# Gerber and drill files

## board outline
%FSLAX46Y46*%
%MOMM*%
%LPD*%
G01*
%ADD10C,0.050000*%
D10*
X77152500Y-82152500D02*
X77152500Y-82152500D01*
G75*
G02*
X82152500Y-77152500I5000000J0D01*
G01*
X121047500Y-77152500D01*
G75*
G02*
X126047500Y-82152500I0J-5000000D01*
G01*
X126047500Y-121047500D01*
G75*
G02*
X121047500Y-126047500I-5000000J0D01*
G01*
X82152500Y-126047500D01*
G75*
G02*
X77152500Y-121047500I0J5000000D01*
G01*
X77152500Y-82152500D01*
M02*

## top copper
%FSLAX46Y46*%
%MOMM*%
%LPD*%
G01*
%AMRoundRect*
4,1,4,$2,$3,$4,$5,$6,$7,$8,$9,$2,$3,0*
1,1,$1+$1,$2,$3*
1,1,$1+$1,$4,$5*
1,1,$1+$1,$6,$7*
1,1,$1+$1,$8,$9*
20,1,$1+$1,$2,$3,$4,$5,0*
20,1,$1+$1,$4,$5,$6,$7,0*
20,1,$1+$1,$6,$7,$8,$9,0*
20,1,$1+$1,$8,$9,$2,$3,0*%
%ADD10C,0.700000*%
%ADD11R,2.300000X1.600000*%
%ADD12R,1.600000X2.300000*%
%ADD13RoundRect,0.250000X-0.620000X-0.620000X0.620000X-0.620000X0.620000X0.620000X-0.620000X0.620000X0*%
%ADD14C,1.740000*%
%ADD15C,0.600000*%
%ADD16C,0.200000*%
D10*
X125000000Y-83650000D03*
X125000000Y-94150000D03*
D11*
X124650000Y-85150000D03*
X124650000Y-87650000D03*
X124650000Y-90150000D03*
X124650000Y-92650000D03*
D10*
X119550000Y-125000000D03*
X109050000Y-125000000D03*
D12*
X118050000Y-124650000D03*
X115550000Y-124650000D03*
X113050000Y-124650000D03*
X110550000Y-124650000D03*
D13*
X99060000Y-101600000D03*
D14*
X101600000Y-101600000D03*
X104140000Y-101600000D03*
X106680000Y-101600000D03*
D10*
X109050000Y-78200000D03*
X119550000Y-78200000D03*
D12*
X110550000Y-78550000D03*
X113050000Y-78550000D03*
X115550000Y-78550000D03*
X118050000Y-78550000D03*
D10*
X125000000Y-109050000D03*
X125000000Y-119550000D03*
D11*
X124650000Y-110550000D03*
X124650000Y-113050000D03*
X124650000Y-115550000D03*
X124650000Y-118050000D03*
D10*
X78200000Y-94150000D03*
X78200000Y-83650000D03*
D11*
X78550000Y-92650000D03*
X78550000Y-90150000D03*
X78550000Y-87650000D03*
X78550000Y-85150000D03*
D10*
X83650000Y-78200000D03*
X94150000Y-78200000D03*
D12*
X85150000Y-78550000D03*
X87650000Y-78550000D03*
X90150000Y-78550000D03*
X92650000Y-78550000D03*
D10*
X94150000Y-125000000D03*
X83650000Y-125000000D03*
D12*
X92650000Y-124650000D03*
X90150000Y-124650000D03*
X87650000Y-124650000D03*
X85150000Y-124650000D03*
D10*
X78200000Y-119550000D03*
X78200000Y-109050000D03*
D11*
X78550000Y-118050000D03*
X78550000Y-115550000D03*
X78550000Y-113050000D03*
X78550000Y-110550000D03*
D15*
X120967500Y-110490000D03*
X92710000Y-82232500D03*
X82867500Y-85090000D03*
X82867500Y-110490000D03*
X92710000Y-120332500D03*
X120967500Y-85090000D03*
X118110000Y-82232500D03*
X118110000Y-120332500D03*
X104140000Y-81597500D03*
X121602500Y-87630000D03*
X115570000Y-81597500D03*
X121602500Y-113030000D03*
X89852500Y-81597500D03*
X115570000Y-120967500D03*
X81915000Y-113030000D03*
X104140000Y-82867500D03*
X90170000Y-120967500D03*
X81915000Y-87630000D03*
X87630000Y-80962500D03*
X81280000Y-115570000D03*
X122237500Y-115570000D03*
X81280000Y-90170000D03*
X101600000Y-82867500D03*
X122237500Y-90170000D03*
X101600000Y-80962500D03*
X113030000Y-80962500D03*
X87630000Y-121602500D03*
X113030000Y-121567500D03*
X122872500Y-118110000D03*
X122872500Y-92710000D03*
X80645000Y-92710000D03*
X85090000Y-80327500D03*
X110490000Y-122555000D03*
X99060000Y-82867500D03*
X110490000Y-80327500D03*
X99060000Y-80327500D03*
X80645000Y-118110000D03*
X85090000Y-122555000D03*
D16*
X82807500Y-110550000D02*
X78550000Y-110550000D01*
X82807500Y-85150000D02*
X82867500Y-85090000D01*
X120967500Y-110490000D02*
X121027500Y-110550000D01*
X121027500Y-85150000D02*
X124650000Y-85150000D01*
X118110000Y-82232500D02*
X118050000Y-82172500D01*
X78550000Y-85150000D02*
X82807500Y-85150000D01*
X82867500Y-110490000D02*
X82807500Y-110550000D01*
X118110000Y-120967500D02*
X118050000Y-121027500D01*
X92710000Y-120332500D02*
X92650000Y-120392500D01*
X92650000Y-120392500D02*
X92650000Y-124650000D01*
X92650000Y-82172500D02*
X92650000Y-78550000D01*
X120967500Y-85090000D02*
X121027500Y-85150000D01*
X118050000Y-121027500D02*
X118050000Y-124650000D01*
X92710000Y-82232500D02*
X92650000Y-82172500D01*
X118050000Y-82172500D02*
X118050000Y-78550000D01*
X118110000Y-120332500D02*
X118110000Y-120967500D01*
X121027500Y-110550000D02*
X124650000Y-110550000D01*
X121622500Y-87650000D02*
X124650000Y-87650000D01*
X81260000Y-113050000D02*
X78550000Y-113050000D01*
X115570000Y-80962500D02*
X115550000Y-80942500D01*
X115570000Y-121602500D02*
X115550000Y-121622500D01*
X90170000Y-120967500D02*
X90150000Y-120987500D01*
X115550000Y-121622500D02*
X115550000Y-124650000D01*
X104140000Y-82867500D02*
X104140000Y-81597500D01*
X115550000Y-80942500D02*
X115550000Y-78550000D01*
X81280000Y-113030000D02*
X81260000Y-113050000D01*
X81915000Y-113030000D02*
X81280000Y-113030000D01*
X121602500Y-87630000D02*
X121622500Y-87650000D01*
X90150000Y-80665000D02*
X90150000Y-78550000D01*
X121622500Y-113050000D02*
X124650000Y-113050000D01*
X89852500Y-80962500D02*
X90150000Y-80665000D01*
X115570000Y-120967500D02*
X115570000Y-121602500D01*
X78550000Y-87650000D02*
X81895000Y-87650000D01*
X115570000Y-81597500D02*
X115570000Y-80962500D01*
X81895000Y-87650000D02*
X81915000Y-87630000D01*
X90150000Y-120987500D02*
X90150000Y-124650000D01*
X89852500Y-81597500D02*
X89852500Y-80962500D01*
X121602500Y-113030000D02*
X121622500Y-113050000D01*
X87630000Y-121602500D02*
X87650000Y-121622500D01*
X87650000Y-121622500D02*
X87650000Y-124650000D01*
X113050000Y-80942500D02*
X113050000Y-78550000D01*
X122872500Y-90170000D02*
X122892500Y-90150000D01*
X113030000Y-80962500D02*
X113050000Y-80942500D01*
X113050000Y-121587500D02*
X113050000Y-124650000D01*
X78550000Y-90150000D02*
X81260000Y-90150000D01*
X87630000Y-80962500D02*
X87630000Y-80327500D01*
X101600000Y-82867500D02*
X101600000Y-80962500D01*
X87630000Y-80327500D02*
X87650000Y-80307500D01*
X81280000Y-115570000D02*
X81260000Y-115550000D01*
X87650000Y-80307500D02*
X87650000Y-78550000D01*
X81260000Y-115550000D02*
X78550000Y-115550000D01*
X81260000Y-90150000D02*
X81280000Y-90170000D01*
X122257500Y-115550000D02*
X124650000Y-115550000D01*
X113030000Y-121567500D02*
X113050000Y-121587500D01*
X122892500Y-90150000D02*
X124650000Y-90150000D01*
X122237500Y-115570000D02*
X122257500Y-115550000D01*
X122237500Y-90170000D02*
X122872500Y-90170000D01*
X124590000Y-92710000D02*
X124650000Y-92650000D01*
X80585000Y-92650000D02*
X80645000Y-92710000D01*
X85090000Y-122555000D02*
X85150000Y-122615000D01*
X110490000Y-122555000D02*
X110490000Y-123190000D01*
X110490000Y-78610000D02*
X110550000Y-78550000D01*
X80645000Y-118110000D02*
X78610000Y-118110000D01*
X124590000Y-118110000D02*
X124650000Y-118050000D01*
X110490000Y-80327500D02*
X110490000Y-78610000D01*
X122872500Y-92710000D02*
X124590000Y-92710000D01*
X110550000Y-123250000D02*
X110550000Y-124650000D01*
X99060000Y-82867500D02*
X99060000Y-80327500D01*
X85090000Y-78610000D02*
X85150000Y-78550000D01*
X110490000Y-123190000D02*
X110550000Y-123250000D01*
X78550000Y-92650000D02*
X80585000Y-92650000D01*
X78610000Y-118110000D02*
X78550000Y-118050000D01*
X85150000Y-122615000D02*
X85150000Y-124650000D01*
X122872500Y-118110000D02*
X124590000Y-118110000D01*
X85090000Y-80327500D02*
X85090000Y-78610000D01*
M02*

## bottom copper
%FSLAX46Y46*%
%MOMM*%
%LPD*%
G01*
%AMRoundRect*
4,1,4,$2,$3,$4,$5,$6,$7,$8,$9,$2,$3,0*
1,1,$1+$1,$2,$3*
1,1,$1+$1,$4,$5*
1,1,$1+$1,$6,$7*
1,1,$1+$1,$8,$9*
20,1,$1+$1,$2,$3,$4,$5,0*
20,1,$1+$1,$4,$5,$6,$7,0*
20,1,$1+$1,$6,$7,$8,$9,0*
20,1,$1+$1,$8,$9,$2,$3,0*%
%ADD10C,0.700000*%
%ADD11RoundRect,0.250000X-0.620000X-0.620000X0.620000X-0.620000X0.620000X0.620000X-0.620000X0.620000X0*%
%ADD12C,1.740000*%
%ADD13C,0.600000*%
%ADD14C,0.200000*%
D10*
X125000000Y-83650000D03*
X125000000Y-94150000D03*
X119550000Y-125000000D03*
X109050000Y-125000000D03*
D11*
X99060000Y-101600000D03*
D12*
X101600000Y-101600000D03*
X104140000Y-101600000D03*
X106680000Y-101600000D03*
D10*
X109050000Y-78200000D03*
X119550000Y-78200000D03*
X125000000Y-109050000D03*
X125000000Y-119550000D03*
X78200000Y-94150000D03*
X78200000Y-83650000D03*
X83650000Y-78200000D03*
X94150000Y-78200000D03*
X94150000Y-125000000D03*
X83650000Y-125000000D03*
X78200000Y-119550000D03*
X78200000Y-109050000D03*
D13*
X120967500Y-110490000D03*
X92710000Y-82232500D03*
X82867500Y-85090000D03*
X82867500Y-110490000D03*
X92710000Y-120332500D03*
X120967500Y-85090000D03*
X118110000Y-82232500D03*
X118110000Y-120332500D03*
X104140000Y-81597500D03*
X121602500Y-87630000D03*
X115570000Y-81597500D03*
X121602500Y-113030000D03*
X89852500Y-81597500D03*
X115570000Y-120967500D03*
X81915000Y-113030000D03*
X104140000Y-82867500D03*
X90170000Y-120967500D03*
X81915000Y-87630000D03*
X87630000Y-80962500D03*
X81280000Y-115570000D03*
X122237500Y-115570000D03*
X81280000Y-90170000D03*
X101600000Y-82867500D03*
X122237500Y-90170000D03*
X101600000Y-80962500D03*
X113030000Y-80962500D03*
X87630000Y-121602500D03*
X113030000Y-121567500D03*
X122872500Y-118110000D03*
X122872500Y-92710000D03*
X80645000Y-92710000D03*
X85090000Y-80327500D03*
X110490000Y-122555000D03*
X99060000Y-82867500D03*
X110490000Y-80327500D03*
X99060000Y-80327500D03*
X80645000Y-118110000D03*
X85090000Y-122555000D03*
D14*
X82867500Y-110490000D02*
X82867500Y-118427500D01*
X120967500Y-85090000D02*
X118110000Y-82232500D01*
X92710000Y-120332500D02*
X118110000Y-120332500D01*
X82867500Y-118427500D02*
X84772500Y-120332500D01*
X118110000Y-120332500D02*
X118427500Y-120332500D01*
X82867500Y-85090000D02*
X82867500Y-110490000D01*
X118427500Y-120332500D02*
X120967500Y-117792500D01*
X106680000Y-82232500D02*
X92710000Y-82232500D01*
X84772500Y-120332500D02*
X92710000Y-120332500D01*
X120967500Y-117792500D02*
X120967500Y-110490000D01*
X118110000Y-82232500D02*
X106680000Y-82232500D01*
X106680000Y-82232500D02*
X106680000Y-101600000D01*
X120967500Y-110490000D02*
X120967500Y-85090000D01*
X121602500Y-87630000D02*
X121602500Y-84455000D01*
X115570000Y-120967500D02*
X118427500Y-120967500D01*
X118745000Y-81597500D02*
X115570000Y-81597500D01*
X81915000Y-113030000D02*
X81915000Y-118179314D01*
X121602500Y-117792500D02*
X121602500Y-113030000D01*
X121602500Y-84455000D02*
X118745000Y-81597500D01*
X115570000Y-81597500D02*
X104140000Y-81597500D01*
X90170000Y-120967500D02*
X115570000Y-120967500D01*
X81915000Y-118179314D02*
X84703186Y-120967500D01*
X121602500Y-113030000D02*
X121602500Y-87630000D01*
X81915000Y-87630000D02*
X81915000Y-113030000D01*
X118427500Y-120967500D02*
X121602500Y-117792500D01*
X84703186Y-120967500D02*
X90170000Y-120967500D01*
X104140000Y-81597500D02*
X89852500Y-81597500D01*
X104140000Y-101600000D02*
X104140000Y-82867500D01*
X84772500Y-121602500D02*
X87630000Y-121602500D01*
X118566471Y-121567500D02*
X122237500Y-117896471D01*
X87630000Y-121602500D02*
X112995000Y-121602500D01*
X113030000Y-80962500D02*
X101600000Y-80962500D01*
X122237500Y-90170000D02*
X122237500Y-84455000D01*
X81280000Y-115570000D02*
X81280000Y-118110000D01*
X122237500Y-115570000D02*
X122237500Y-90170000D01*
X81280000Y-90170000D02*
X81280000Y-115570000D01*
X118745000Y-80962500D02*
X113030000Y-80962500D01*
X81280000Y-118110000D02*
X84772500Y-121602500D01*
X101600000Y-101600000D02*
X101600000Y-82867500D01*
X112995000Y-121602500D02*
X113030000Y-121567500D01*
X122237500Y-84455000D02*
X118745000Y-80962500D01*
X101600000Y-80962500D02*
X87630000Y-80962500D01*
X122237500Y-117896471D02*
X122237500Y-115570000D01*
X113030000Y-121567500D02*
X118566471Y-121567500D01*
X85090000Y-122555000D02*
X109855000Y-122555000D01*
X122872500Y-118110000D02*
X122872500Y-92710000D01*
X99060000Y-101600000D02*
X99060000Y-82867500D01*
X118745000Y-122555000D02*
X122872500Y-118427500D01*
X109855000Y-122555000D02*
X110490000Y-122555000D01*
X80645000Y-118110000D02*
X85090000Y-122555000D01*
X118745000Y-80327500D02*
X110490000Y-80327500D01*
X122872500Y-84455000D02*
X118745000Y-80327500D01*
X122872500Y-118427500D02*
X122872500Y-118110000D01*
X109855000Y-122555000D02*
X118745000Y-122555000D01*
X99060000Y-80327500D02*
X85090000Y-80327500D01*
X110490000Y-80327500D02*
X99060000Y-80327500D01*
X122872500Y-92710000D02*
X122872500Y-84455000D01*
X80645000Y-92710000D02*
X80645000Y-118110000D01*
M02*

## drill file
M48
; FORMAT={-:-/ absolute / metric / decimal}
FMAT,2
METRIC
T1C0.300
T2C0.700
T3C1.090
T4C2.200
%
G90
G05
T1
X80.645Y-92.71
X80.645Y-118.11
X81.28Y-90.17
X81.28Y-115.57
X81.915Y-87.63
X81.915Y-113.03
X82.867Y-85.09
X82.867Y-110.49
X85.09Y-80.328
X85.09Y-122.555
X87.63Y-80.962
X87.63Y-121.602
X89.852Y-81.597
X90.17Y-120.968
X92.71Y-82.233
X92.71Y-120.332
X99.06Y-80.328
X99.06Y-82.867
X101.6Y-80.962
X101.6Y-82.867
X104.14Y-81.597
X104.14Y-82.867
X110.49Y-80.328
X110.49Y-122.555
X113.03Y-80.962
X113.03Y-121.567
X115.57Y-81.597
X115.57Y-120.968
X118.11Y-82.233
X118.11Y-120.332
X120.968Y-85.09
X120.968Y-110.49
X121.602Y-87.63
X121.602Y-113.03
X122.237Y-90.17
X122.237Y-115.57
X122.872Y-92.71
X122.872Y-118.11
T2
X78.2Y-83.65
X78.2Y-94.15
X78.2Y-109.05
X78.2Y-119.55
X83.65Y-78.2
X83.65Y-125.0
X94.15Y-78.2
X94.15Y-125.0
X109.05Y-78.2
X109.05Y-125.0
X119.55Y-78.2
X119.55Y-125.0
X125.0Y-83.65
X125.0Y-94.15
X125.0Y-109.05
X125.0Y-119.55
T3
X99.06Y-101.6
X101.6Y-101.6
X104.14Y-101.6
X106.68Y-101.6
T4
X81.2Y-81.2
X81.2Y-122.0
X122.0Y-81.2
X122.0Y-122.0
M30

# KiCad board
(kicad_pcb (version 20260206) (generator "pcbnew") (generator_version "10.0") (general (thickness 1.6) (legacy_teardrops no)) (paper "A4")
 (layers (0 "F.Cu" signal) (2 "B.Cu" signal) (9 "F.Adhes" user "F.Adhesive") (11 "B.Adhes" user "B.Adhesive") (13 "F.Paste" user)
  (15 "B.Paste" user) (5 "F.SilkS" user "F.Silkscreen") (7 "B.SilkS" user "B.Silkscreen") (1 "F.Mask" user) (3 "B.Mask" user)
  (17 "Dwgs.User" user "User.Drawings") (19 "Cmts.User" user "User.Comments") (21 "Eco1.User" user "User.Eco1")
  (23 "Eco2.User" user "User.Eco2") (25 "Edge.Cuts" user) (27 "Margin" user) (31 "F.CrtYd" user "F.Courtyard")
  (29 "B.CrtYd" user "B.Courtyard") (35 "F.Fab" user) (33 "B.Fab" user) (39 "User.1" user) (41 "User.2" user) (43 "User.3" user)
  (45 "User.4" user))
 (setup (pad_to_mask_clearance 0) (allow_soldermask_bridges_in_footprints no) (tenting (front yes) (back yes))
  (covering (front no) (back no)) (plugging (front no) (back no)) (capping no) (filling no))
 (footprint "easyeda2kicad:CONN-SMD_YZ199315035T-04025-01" (layer "F.Cu") (at 124.65 88.9 -90)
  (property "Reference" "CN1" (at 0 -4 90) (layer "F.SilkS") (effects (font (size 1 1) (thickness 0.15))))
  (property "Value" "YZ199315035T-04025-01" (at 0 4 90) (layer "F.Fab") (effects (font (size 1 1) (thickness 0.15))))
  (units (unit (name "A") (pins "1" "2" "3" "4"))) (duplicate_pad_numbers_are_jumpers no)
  (pad "" thru_hole circle (at -5.25 -0.35 270) (size 0.7 0.7) (drill 0.7) (layers "*.Cu" "*.Mask") (remove_unused_layers no))
  (pad "" thru_hole circle (at 5.25 -0.35 270) (size 0.7 0.7) (drill 0.7) (layers "*.Cu" "*.Mask") (remove_unused_layers no))
  (pad "1" smd rect (at -3.75 0 270) (size 1.6 2.3) (layers "F.Cu" "F.Mask" "F.Paste") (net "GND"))
  (pad "2" smd rect (at -1.25 0 270) (size 1.6 2.3) (layers "F.Cu" "F.Mask" "F.Paste") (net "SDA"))
  (pad "3" smd rect (at 1.25 0 270) (size 1.6 2.3) (layers "F.Cu" "F.Mask" "F.Paste") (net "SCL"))
  (pad "4" smd rect (at 3.75 0 270) (size 1.6 2.3) (layers "F.Cu" "F.Mask" "F.Paste") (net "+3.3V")))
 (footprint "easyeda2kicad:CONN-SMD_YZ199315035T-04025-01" (layer "F.Cu") (at 114.3 124.65 180)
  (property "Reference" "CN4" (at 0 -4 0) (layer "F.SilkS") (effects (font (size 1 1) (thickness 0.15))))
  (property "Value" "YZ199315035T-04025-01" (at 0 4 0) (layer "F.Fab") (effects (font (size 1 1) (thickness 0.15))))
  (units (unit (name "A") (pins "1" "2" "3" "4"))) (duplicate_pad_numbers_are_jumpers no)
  (pad "" thru_hole circle (at -5.25 -0.35 180) (size 0.7 0.7) (drill 0.7) (layers "*.Cu" "*.Mask") (remove_unused_layers no))
  (pad "" thru_hole circle (at 5.25 -0.35 180) (size 0.7 0.7) (drill 0.7) (layers "*.Cu" "*.Mask") (remove_unused_layers no))
  (pad "1" smd rect (at -3.75 0 180) (size 1.6 2.3) (layers "F.Cu" "F.Mask" "F.Paste") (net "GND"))
  (pad "2" smd rect (at -1.25 0 180) (size 1.6 2.3) (layers "F.Cu" "F.Mask" "F.Paste") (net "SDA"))
  (pad "3" smd rect (at 1.25 0 180) (size 1.6 2.3) (layers "F.Cu" "F.Mask" "F.Paste") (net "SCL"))
  (pad "4" smd rect (at 3.75 0 180) (size 1.6 2.3) (layers "F.Cu" "F.Mask" "F.Paste") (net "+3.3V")))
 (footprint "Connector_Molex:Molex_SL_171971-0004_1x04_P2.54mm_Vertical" (layer "F.Cu") (at 99.06 101.6)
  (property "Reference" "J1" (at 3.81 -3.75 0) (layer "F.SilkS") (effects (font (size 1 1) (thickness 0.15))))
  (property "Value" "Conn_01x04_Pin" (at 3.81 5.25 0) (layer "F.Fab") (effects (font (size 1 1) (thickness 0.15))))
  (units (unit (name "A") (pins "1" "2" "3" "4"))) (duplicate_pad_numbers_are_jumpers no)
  (pad "1" thru_hole roundrect (at 0 0) (size 1.74 1.74) (drill 1.09) (layers "*.Cu" "*.Mask") (remove_unused_layers no)
   (roundrect_rratio 0.143678) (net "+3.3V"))
  (pad "2" thru_hole circle (at 2.54 0) (size 1.74 1.74) (drill 1.09) (layers "*.Cu" "*.Mask") (remove_unused_layers no) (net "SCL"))
  (pad "3" thru_hole circle (at 5.08 0) (size 1.74 1.74) (drill 1.09) (layers "*.Cu" "*.Mask") (remove_unused_layers no) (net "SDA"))
  (pad "4" thru_hole circle (at 7.62 0) (size 1.74 1.74) (drill 1.09) (layers "*.Cu" "*.Mask") (remove_unused_layers no) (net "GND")))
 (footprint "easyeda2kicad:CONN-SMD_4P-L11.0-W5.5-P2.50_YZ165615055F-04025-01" (layer "F.Cu") (at 114.3 78.55)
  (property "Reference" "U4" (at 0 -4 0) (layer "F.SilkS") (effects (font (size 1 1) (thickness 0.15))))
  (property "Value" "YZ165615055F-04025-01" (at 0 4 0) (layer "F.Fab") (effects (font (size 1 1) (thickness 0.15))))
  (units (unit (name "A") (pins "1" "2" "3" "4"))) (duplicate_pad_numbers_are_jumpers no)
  (pad "" thru_hole circle (at -5.25 -0.35) (size 0.7 0.7) (drill 0.7) (layers "*.Cu" "*.Mask") (remove_unused_layers no))
  (pad "" thru_hole circle (at 5.25 -0.35) (size 0.7 0.7) (drill 0.7) (layers "*.Cu" "*.Mask") (remove_unused_layers no))
  (pad "1" smd rect (at -3.75 0) (size 1.6 2.3) (layers "F.Cu" "F.Mask" "F.Paste") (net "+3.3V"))
  (pad "2" smd rect (at -1.25 0) (size 1.6 2.3) (layers "F.Cu" "F.Mask" "F.Paste") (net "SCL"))
  (pad "3" smd rect (at 1.25 0) (size 1.6 2.3) (layers "F.Cu" "F.Mask" "F.Paste") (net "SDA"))
  (pad "4" smd rect (at 3.75 0) (size 1.6 2.3) (layers "F.Cu" "F.Mask" "F.Paste") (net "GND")))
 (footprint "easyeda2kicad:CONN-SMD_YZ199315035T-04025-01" (layer "F.Cu") (at 124.65 114.3 -90)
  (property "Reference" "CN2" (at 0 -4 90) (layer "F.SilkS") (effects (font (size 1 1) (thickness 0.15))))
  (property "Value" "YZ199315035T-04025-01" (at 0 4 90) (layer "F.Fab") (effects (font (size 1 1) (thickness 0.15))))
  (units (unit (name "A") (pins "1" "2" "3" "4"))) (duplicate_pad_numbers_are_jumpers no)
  (pad "" thru_hole circle (at -5.25 -0.35 270) (size 0.7 0.7) (drill 0.7) (layers "*.Cu" "*.Mask") (remove_unused_layers no))
  (pad "" thru_hole circle (at 5.25 -0.35 270) (size 0.7 0.7) (drill 0.7) (layers "*.Cu" "*.Mask") (remove_unused_layers no))
  (pad "1" smd rect (at -3.75 0 270) (size 1.6 2.3) (layers "F.Cu" "F.Mask" "F.Paste") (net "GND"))
  (pad "2" smd rect (at -1.25 0 270) (size 1.6 2.3) (layers "F.Cu" "F.Mask" "F.Paste") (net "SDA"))
  (pad "3" smd rect (at 1.25 0 270) (size 1.6 2.3) (layers "F.Cu" "F.Mask" "F.Paste") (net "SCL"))
  (pad "4" smd rect (at 3.75 0 270) (size 1.6 2.3) (layers "F.Cu" "F.Mask" "F.Paste") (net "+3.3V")))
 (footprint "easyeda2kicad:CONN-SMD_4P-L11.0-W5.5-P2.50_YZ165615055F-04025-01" (layer "F.Cu") (at 78.55 88.9 90)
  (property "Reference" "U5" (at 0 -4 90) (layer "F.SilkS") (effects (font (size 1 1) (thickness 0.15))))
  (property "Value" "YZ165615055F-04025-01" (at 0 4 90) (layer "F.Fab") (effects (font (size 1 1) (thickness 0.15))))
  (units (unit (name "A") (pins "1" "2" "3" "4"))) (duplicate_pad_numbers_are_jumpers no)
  (pad "" thru_hole circle (at -5.25 -0.35 90) (size 0.7 0.7) (drill 0.7) (layers "*.Cu" "*.Mask") (remove_unused_layers no))
  (pad "" thru_hole circle (at 5.25 -0.35 90) (size 0.7 0.7) (drill 0.7) (layers "*.Cu" "*.Mask") (remove_unused_layers no))
  (pad "1" smd rect (at -3.75 0 90) (size 1.6 2.3) (layers "F.Cu" "F.Mask" "F.Paste") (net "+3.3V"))
  (pad "2" smd rect (at -1.25 0 90) (size 1.6 2.3) (layers "F.Cu" "F.Mask" "F.Paste") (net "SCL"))
  (pad "3" smd rect (at 1.25 0 90) (size 1.6 2.3) (layers "F.Cu" "F.Mask" "F.Paste") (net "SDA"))
  (pad "4" smd rect (at 3.75 0 90) (size 1.6 2.3) (layers "F.Cu" "F.Mask" "F.Paste") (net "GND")))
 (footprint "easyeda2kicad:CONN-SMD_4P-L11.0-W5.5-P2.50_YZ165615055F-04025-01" (layer "F.Cu") (at 88.9 78.55)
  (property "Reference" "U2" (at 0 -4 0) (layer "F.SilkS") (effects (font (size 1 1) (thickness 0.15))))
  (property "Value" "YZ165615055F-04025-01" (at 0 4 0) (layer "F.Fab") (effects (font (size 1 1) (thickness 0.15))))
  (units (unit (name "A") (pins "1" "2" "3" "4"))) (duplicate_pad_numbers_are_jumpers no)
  (pad "" thru_hole circle (at -5.25 -0.35) (size 0.7 0.7) (drill 0.7) (layers "*.Cu" "*.Mask") (remove_unused_layers no))
  (pad "" thru_hole circle (at 5.25 -0.35) (size 0.7 0.7) (drill 0.7) (layers "*.Cu" "*.Mask") (remove_unused_layers no))
  (pad "1" smd rect (at -3.75 0) (size 1.6 2.3) (layers "F.Cu" "F.Mask" "F.Paste") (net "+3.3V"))
  (pad "2" smd rect (at -1.25 0) (size 1.6 2.3) (layers "F.Cu" "F.Mask" "F.Paste") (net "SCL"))
  (pad "3" smd rect (at 1.25 0) (size 1.6 2.3) (layers "F.Cu" "F.Mask" "F.Paste") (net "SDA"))
  (pad "4" smd rect (at 3.75 0) (size 1.6 2.3) (layers "F.Cu" "F.Mask" "F.Paste") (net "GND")))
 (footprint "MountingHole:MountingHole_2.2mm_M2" (layer "F.Cu") (at 122 81.2)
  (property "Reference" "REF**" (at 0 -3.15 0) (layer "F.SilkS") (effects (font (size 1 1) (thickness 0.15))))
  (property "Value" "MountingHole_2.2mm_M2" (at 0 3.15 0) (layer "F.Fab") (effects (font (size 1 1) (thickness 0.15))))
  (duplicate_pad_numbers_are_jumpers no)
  (pad "" np_thru_hole circle (at 0 0) (size 2.2 2.2) (drill 2.2) (layers "*.Cu" "*.Mask")))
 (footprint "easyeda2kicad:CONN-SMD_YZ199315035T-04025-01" (layer "F.Cu") (at 88.9 124.65 180)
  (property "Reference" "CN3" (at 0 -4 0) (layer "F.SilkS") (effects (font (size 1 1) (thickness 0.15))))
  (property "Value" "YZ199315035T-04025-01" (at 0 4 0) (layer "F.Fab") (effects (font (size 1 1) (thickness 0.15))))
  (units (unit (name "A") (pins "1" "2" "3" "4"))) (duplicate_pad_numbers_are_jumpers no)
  (pad "" thru_hole circle (at -5.25 -0.35 180) (size 0.7 0.7) (drill 0.7) (layers "*.Cu" "*.Mask") (remove_unused_layers no))
  (pad "" thru_hole circle (at 5.25 -0.35 180) (size 0.7 0.7) (drill 0.7) (layers "*.Cu" "*.Mask") (remove_unused_layers no))
  (pad "1" smd rect (at -3.75 0 180) (size 1.6 2.3) (layers "F.Cu" "F.Mask" "F.Paste") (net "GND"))
  (pad "2" smd rect (at -1.25 0 180) (size 1.6 2.3) (layers "F.Cu" "F.Mask" "F.Paste") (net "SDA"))
  (pad "3" smd rect (at 1.25 0 180) (size 1.6 2.3) (layers "F.Cu" "F.Mask" "F.Paste") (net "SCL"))
  (pad "4" smd rect (at 3.75 0 180) (size 1.6 2.3) (layers "F.Cu" "F.Mask" "F.Paste") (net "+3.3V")))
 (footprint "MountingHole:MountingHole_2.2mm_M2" (layer "F.Cu") (at 81.2 81.2)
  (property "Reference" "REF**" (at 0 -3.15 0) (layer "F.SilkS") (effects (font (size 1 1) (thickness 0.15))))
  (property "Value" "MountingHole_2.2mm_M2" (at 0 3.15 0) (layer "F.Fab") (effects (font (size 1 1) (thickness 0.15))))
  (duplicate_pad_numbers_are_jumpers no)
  (pad "" np_thru_hole circle (at 0 0) (size 2.2 2.2) (drill 2.2) (layers "*.Cu" "*.Mask")))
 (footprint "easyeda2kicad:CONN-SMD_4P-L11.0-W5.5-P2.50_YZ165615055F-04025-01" (layer "F.Cu") (at 78.55 114.3 90)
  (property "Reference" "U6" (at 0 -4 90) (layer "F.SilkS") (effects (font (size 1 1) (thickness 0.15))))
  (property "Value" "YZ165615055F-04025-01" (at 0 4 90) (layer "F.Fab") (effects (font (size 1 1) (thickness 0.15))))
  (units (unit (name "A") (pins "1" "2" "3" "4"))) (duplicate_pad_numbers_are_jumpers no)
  (pad "" thru_hole circle (at -5.25 -0.35 90) (size 0.7 0.7) (drill 0.7) (layers "*.Cu" "*.Mask") (remove_unused_layers no))
  (pad "" thru_hole circle (at 5.25 -0.35 90) (size 0.7 0.7) (drill 0.7) (layers "*.Cu" "*.Mask") (remove_unused_layers no))
  (pad "1" smd rect (at -3.75 0 90) (size 1.6 2.3) (layers "F.Cu" "F.Mask" "F.Paste") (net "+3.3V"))
  (pad "2" smd rect (at -1.25 0 90) (size 1.6 2.3) (layers "F.Cu" "F.Mask" "F.Paste") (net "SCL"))
  (pad "3" smd rect (at 1.25 0 90) (size 1.6 2.3) (layers "F.Cu" "F.Mask" "F.Paste") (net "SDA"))
  (pad "4" smd rect (at 3.75 0 90) (size 1.6 2.3) (layers "F.Cu" "F.Mask" "F.Paste") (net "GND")))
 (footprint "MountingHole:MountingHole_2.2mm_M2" (layer "F.Cu") (at 81.2 122)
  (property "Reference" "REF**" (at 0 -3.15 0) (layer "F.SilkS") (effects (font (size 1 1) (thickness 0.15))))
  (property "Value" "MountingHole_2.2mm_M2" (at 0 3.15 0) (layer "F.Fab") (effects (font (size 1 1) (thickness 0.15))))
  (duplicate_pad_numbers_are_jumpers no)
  (pad "" np_thru_hole circle (at 0 0) (size 2.2 2.2) (drill 2.2) (layers "*.Cu" "*.Mask")))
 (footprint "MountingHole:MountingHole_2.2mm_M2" (layer "F.Cu") (at 122 122)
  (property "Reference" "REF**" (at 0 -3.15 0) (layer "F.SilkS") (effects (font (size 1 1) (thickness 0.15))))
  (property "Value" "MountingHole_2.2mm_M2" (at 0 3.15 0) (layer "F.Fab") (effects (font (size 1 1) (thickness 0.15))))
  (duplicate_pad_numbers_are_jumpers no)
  (pad "" np_thru_hole circle (at 0 0) (size 2.2 2.2) (drill 2.2) (layers "*.Cu" "*.Mask")))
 (gr_rect (start 77.1525 77.1525) (end 126.0475 126.0475) (radius 5) (stroke (width 0.05) (type solid)) (fill no) (layer "Edge.Cuts"))
 (segment (start 82.8075 110.55) (end 78.55 110.55) (width 0.2) (layer "F.Cu") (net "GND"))
 (segment (start 82.8075 85.15) (end 82.8675 85.09) (width 0.2) (layer "F.Cu") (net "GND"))
 (segment (start 120.9675 110.49) (end 121.0275 110.55) (width 0.2) (layer "F.Cu") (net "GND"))
 (segment (start 121.0275 85.15) (end 124.65 85.15) (width 0.2) (layer "F.Cu") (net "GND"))
 (segment (start 118.11 82.2325) (end 118.05 82.1725) (width 0.2) (layer "F.Cu") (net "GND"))
 (segment (start 78.55 85.15) (end 82.8075 85.15) (width 0.2) (layer "F.Cu") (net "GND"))
 (segment (start 82.8675 110.49) (end 82.8075 110.55) (width 0.2) (layer "F.Cu") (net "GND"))
 (segment (start 118.11 120.9675) (end 118.05 121.0275) (width 0.2) (layer "F.Cu") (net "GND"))
 (segment (start 92.71 120.3325) (end 92.65 120.3925) (width 0.2) (layer "F.Cu") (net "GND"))
 (segment (start 92.65 120.3925) (end 92.65 124.65) (width 0.2) (layer "F.Cu") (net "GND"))
 (segment (start 92.65 82.1725) (end 92.65 78.55) (width 0.2) (layer "F.Cu") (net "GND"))
 (segment (start 120.9675 85.09) (end 121.0275 85.15) (width 0.2) (layer "F.Cu") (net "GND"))
 (segment (start 118.05 121.0275) (end 118.05 124.65) (width 0.2) (layer "F.Cu") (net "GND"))
 (segment (start 92.71 82.2325) (end 92.65 82.1725) (width 0.2) (layer "F.Cu") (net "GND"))
 (segment (start 118.05 82.1725) (end 118.05 78.55) (width 0.2) (layer "F.Cu") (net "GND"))
 (segment (start 118.11 120.3325) (end 118.11 120.9675) (width 0.2) (layer "F.Cu") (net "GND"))
 (segment (start 121.0275 110.55) (end 124.65 110.55) (width 0.2) (layer "F.Cu") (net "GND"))
 (via (at 120.9675 110.49) (size 0.6) (drill 0.3) (layers "F.Cu" "B.Cu") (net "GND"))
 (via (at 92.71 82.2325) (size 0.6) (drill 0.3) (layers "F.Cu" "B.Cu") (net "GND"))
 (via (at 82.8675 85.09) (size 0.6) (drill 0.3) (layers "F.Cu" "B.Cu") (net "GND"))
 (via (at 82.8675 110.49) (size 0.6) (drill 0.3) (layers "F.Cu" "B.Cu") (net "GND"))
 (via (at 92.71 120.3325) (size 0.6) (drill 0.3) (layers "F.Cu" "B.Cu") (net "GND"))
 (via (at 120.9675 85.09) (size 0.6) (drill 0.3) (layers "F.Cu" "B.Cu") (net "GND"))
 (via (at 118.11 82.2325) (size 0.6) (drill 0.3) (layers "F.Cu" "B.Cu") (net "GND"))
 (via (at 118.11 120.3325) (size 0.6) (drill 0.3) (layers "F.Cu" "B.Cu") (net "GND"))
 (segment (start 82.8675 110.49) (end 82.8675 118.4275) (width 0.2) (layer "B.Cu") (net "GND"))
 (segment (start 120.9675 85.09) (end 118.11 82.2325) (width 0.2) (layer "B.Cu") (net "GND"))
 (segment (start 92.71 120.3325) (end 118.11 120.3325) (width 0.2) (layer "B.Cu") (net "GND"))
 (segment (start 82.8675 118.4275) (end 84.7725 120.3325) (width 0.2) (layer "B.Cu") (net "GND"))
 (segment (start 118.11 120.3325) (end 118.4275 120.3325) (width 0.2) (layer "B.Cu") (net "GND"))
 (segment (start 82.8675 85.09) (end 82.8675 110.49) (width 0.2) (layer "B.Cu") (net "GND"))
 (segment (start 118.4275 120.3325) (end 120.9675 117.7925) (width 0.2) (layer "B.Cu") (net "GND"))
 (segment (start 106.68 82.2325) (end 92.71 82.2325) (width 0.2) (layer "B.Cu") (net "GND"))
 (segment (start 84.7725 120.3325) (end 92.71 120.3325) (width 0.2) (layer "B.Cu") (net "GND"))
 (segment (start 120.9675 117.7925) (end 120.9675 110.49) (width 0.2) (layer "B.Cu") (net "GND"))
 (segment (start 118.11 82.2325) (end 106.68 82.2325) (width 0.2) (layer "B.Cu") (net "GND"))
 (segment (start 106.68 82.2325) (end 106.68 101.6) (width 0.2) (layer "B.Cu") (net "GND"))
 (segment (start 120.9675 110.49) (end 120.9675 85.09) (width 0.2) (layer "B.Cu") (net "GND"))
 (segment (start 121.6225 87.65) (end 124.65 87.65) (width 0.2) (layer "F.Cu") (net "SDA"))
 (segment (start 81.26 113.05) (end 78.55 113.05) (width 0.2) (layer "F.Cu") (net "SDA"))
 (segment (start 115.57 80.9625) (end 115.55 80.9425) (width 0.2) (layer "F.Cu") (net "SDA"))
 (segment (start 115.57 121.6025) (end 115.55 121.6225) (width 0.2) (layer "F.Cu") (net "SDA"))
 (segment (start 90.17 120.9675) (end 90.15 120.9875) (width 0.2) (layer "F.Cu") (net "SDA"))
 (segment (start 115.55 121.6225) (end 115.55 124.65) (width 0.2) (layer "F.Cu") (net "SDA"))
 (segment (start 104.14 82.8675) (end 104.14 81.5975) (width 0.2) (layer "F.Cu") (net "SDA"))
 (segment (start 115.55 80.9425) (end 115.55 78.55) (width 0.2) (layer "F.Cu") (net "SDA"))
 (segment (start 81.28 113.03) (end 81.26 113.05) (width 0.2) (layer "F.Cu") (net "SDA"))
 (segment (start 81.915 113.03) (end 81.28 113.03) (width 0.2) (layer "F.Cu") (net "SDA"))
 (segment (start 121.6025 87.63) (end 121.6225 87.65) (width 0.2) (layer "F.Cu") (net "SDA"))
 (segment (start 90.15 80.665) (end 90.15 78.55) (width 0.2) (layer "F.Cu") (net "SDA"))
 (segment (start 121.6225 113.05) (end 124.65 113.05) (width 0.2) (layer "F.Cu") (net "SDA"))
 (segment (start 89.8525 80.9625) (end 90.15 80.665) (width 0.2) (layer "F.Cu") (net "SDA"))
 (segment (start 115.57 120.9675) (end 115.57 121.6025) (width 0.2) (layer "F.Cu") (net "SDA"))
 (segment (start 78.55 87.65) (end 81.895 87.65) (width 0.2) (layer "F.Cu") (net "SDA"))
 (segment (start 115.57 81.5975) (end 115.57 80.9625) (width 0.2) (layer "F.Cu") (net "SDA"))
 (segment (start 81.895 87.65) (end 81.915 87.63) (width 0.2) (layer "F.Cu") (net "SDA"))
 (segment (start 90.15 120.9875) (end 90.15 124.65) (width 0.2) (layer "F.Cu") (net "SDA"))
 (segment (start 89.8525 81.5975) (end 89.8525 80.9625) (width 0.2) (layer "F.Cu") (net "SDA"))
 (segment (start 121.6025 113.03) (end 121.6225 113.05) (width 0.2) (layer "F.Cu") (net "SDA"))
 (via (at 104.14 81.5975) (size 0.6) (drill 0.3) (layers "F.Cu" "B.Cu") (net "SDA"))
 (via (at 121.6025 87.63) (size 0.6) (drill 0.3) (layers "F.Cu" "B.Cu") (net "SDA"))
 (via (at 115.57 81.5975) (size 0.6) (drill 0.3) (layers "F.Cu" "B.Cu") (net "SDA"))
 (via (at 121.6025 113.03) (size 0.6) (drill 0.3) (layers "F.Cu" "B.Cu") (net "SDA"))
 (via (at 89.8525 81.5975) (size 0.6) (drill 0.3) (layers "F.Cu" "B.Cu") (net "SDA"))
 (via (at 115.57 120.9675) (size 0.6) (drill 0.3) (layers "F.Cu" "B.Cu") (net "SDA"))
 (via (at 81.915 113.03) (size 0.6) (drill 0.3) (layers "F.Cu" "B.Cu") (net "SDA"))
 (via (at 104.14 82.8675) (size 0.6) (drill 0.3) (layers "F.Cu" "B.Cu") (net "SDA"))
 (via (at 90.17 120.9675) (size 0.6) (drill 0.3) (layers "F.Cu" "B.Cu") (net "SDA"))
 (via (at 81.915 87.63) (size 0.6) (drill 0.3) (layers "F.Cu" "B.Cu") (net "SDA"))
 (segment (start 121.6025 87.63) (end 121.6025 84.455) (width 0.2) (layer "B.Cu") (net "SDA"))
 (segment (start 115.57 120.9675) (end 118.4275 120.9675) (width 0.2) (layer "B.Cu") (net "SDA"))
 (segment (start 118.745 81.5975) (end 115.57 81.5975) (width 0.2) (layer "B.Cu") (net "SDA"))
 (segment (start 81.915 113.03) (end 81.915 118.179314) (width 0.2) (layer "B.Cu") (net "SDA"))
 (segment (start 121.6025 117.7925) (end 121.6025 113.03) (width 0.2) (layer "B.Cu") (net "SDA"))
 (segment (start 121.6025 84.455) (end 118.745 81.5975) (width 0.2) (layer "B.Cu") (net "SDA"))
 (segment (start 115.57 81.5975) (end 104.14 81.5975) (width 0.2) (layer "B.Cu") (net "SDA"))
 (segment (start 90.17 120.9675) (end 115.57 120.9675) (width 0.2) (layer "B.Cu") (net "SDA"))
 (segment (start 81.915 118.179314) (end 84.703186 120.9675) (width 0.2) (layer "B.Cu") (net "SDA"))
 (segment (start 121.6025 113.03) (end 121.6025 87.63) (width 0.2) (layer "B.Cu") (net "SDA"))
 (segment (start 81.915 87.63) (end 81.915 113.03) (width 0.2) (layer "B.Cu") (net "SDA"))
 (segment (start 118.4275 120.9675) (end 121.6025 117.7925) (width 0.2) (layer "B.Cu") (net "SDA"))
 (segment (start 84.703186 120.9675) (end 90.17 120.9675) (width 0.2) (layer "B.Cu") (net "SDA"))
 (segment (start 104.14 81.5975) (end 89.8525 81.5975) (width 0.2) (layer "B.Cu") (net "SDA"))
 (segment (start 104.14 101.6) (end 104.14 82.8675) (width 0.2) (layer "B.Cu") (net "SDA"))
 (segment (start 87.63 121.6025) (end 87.65 121.6225) (width 0.2) (layer "F.Cu") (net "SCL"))
 (segment (start 87.65 121.6225) (end 87.65 124.65) (width 0.2) (layer "F.Cu") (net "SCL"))
 (segment (start 113.05 80.9425) (end 113.05 78.55) (width 0.2) (layer "F.Cu") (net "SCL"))
 (segment (start 122.8725 90.17) (end 122.8925 90.15) (width 0.2) (layer "F.Cu") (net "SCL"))
 (segment (start 113.03 80.9625) (end 113.05 80.9425) (width 0.2) (layer "F.Cu") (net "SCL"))
 (segment (start 113.05 121.5875) (end 113.05 124.65) (width 0.2) (layer "F.Cu") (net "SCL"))
 (segment (start 78.55 90.15) (end 81.26 90.15) (width 0.2) (layer "F.Cu") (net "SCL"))
 (segment (start 87.63 80.9625) (end 87.63 80.3275) (width 0.2) (layer "F.Cu") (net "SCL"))
 (segment (start 101.6 82.8675) (end 101.6 80.9625) (width 0.2) (layer "F.Cu") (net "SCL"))
 (segment (start 87.63 80.3275) (end 87.65 80.3075) (width 0.2) (layer "F.Cu") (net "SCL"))
 (segment (start 81.28 115.57) (end 81.26 115.55) (width 0.2) (layer "F.Cu") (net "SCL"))
 (segment (start 87.65 80.3075) (end 87.65 78.55) (width 0.2) (layer "F.Cu") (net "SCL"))
 (segment (start 81.26 115.55) (end 78.55 115.55) (width 0.2) (layer "F.Cu") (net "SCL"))
 (segment (start 81.26 90.15) (end 81.28 90.17) (width 0.2) (layer "F.Cu") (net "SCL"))
 (segment (start 122.2575 115.55) (end 124.65 115.55) (width 0.2) (layer "F.Cu") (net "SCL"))
 (segment (start 113.03 121.5675) (end 113.05 121.5875) (width 0.2) (layer "F.Cu") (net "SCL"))
 (segment (start 122.8925 90.15) (end 124.65 90.15) (width 0.2) (layer "F.Cu") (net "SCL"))
 (segment (start 122.2375 115.57) (end 122.2575 115.55) (width 0.2) (layer "F.Cu") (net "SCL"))
 (segment (start 122.2375 90.17) (end 122.8725 90.17) (width 0.2) (layer "F.Cu") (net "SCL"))
 (via (at 87.63 80.9625) (size 0.6) (drill 0.3) (layers "F.Cu" "B.Cu") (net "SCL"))
 (via (at 81.28 115.57) (size 0.6) (drill 0.3) (layers "F.Cu" "B.Cu") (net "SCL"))
 (via (at 122.2375 115.57) (size 0.6) (drill 0.3) (layers "F.Cu" "B.Cu") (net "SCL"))
 (via (at 81.28 90.17) (size 0.6) (drill 0.3) (layers "F.Cu" "B.Cu") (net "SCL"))
 (via (at 101.6 82.8675) (size 0.6) (drill 0.3) (layers "F.Cu" "B.Cu") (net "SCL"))
 (via (at 122.2375 90.17) (size 0.6) (drill 0.3) (layers "F.Cu" "B.Cu") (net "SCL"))
 (via (at 101.6 80.9625) (size 0.6) (drill 0.3) (layers "F.Cu" "B.Cu") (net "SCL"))
 (via (at 113.03 80.9625) (size 0.6) (drill 0.3) (layers "F.Cu" "B.Cu") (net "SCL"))
 (via (at 87.63 121.6025) (size 0.6) (drill 0.3) (layers "F.Cu" "B.Cu") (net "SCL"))
 (via (at 113.03 121.5675) (size 0.6) (drill 0.3) (layers "F.Cu" "B.Cu") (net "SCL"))
 (segment (start 84.7725 121.6025) (end 87.63 121.6025) (width 0.2) (layer "B.Cu") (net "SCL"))
 (segment (start 118.566471 121.5675) (end 122.2375 117.896471) (width 0.2) (layer "B.Cu") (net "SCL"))
 (segment (start 87.63 121.6025) (end 112.995 121.6025) (width 0.2) (layer "B.Cu") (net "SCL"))
 (segment (start 113.03 80.9625) (end 101.6 80.9625) (width 0.2) (layer "B.Cu") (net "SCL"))
 (segment (start 122.2375 90.17) (end 122.2375 84.455) (width 0.2) (layer "B.Cu") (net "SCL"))
 (segment (start 81.28 115.57) (end 81.28 118.11) (width 0.2) (layer "B.Cu") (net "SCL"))
 (segment (start 122.2375 115.57) (end 122.2375 90.17) (width 0.2) (layer "B.Cu") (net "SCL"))
 (segment (start 81.28 90.17) (end 81.28 115.57) (width 0.2) (layer "B.Cu") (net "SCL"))
 (segment (start 118.745 80.9625) (end 113.03 80.9625) (width 0.2) (layer "B.Cu") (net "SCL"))
 (segment (start 81.28 118.11) (end 84.7725 121.6025) (width 0.2) (layer "B.Cu") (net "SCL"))
 (segment (start 101.6 101.6) (end 101.6 82.8675) (width 0.2) (layer "B.Cu") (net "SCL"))
 (segment (start 112.995 121.6025) (end 113.03 121.5675) (width 0.2) (layer "B.Cu") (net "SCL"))
 (segment (start 122.2375 84.455) (end 118.745 80.9625) (width 0.2) (layer "B.Cu") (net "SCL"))
 (segment (start 101.6 80.9625) (end 87.63 80.9625) (width 0.2) (layer "B.Cu") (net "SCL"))
 (segment (start 122.2375 117.896471) (end 122.2375 115.57) (width 0.2) (layer "B.Cu") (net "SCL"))
 (segment (start 113.03 121.5675) (end 118.566471 121.5675) (width 0.2) (layer "B.Cu") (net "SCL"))
 (segment (start 124.59 92.71) (end 124.65 92.65) (width 0.2) (layer "F.Cu") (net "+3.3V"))
 (segment (start 80.585 92.65) (end 80.645 92.71) (width 0.2) (layer "F.Cu") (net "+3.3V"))
 (segment (start 85.09 122.555) (end 85.15 122.615) (width 0.2) (layer "F.Cu") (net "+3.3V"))
 (segment (start 110.49 122.555) (end 110.49 123.19) (width 0.2) (layer "F.Cu") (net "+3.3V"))
 (segment (start 110.49 78.61) (end 110.55 78.55) (width 0.2) (layer "F.Cu") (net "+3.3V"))
 (segment (start 80.645 118.11) (end 78.61 118.11) (width 0.2) (layer "F.Cu") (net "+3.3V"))
 (segment (start 124.59 118.11) (end 124.65 118.05) (width 0.2) (layer "F.Cu") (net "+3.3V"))
 (segment (start 110.49 80.3275) (end 110.49 78.61) (width 0.2) (layer "F.Cu") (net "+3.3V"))
 (segment (start 122.8725 92.71) (end 124.59 92.71) (width 0.2) (layer "F.Cu") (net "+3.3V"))
 (segment (start 110.55 123.25) (end 110.55 124.65) (width 0.2) (layer "F.Cu") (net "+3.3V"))
 (segment (start 99.06 82.8675) (end 99.06 80.3275) (width 0.2) (layer "F.Cu") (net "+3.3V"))
 (segment (start 85.09 78.61) (end 85.15 78.55) (width 0.2) (layer "F.Cu") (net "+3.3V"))
 (segment (start 110.49 123.19) (end 110.55 123.25) (width 0.2) (layer "F.Cu") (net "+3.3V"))
 (segment (start 78.55 92.65) (end 80.585 92.65) (width 0.2) (layer "F.Cu") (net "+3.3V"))
 (segment (start 78.61 118.11) (end 78.55 118.05) (width 0.2) (layer "F.Cu") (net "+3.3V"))
 (segment (start 85.15 122.615) (end 85.15 124.65) (width 0.2) (layer "F.Cu") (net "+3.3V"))
 (segment (start 122.8725 118.11) (end 124.59 118.11) (width 0.2) (layer "F.Cu") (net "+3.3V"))
 (segment (start 85.09 80.3275) (end 85.09 78.61) (width 0.2) (layer "F.Cu") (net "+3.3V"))
 (via (at 122.8725 118.11) (size 0.6) (drill 0.3) (layers "F.Cu" "B.Cu") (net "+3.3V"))
 (via (at 122.8725 92.71) (size 0.6) (drill 0.3) (layers "F.Cu" "B.Cu") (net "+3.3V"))
 (via (at 80.645 92.71) (size 0.6) (drill 0.3) (layers "F.Cu" "B.Cu") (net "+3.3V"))
 (via (at 85.09 80.3275) (size 0.6) (drill 0.3) (layers "F.Cu" "B.Cu") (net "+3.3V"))
 (via (at 110.49 122.555) (size 0.6) (drill 0.3) (layers "F.Cu" "B.Cu") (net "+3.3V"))
 (via (at 99.06 82.8675) (size 0.6) (drill 0.3) (layers "F.Cu" "B.Cu") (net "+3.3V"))
 (via (at 110.49 80.3275) (size 0.6) (drill 0.3) (layers "F.Cu" "B.Cu") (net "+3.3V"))
 (via (at 99.06 80.3275) (size 0.6) (drill 0.3) (layers "F.Cu" "B.Cu") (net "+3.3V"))
 (via (at 80.645 118.11) (size 0.6) (drill 0.3) (layers "F.Cu" "B.Cu") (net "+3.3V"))
 (via (at 85.09 122.555) (size 0.6) (drill 0.3) (layers "F.Cu" "B.Cu") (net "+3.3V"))
 (segment (start 85.09 122.555) (end 109.855 122.555) (width 0.2) (layer "B.Cu") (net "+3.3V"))
 (segment (start 122.8725 118.11) (end 122.8725 92.71) (width 0.2) (layer "B.Cu") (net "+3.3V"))
 (segment (start 99.06 101.6) (end 99.06 82.8675) (width 0.2) (layer "B.Cu") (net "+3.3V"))
 (segment (start 118.745 122.555) (end 122.8725 118.4275) (width 0.2) (layer "B.Cu") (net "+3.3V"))
 (segment (start 109.855 122.555) (end 110.49 122.555) (width 0.2) (layer "B.Cu") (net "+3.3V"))
 (segment (start 80.645 118.11) (end 85.09 122.555) (width 0.2) (layer "B.Cu") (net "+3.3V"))
 (segment (start 118.745 80.3275) (end 110.49 80.3275) (width 0.2) (layer "B.Cu") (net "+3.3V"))
 (segment (start 122.8725 84.455) (end 118.745 80.3275) (width 0.2) (layer "B.Cu") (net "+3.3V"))
 (segment (start 122.8725 118.4275) (end 122.8725 118.11) (width 0.2) (layer "B.Cu") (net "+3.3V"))
 (segment (start 109.855 122.555) (end 118.745 122.555) (width 0.2) (layer "B.Cu") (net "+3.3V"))
 (segment (start 99.06 80.3275) (end 85.09 80.3275) (width 0.2) (layer "B.Cu") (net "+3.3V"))
 (segment (start 110.49 80.3275) (end 99.06 80.3275) (width 0.2) (layer "B.Cu") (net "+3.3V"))
 (segment (start 122.8725 92.71) (end 122.8725 84.455) (width 0.2) (layer "B.Cu") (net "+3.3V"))
 (segment (start 80.645 92.71) (end 80.645 118.11) (width 0.2) (layer "B.Cu") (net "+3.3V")))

